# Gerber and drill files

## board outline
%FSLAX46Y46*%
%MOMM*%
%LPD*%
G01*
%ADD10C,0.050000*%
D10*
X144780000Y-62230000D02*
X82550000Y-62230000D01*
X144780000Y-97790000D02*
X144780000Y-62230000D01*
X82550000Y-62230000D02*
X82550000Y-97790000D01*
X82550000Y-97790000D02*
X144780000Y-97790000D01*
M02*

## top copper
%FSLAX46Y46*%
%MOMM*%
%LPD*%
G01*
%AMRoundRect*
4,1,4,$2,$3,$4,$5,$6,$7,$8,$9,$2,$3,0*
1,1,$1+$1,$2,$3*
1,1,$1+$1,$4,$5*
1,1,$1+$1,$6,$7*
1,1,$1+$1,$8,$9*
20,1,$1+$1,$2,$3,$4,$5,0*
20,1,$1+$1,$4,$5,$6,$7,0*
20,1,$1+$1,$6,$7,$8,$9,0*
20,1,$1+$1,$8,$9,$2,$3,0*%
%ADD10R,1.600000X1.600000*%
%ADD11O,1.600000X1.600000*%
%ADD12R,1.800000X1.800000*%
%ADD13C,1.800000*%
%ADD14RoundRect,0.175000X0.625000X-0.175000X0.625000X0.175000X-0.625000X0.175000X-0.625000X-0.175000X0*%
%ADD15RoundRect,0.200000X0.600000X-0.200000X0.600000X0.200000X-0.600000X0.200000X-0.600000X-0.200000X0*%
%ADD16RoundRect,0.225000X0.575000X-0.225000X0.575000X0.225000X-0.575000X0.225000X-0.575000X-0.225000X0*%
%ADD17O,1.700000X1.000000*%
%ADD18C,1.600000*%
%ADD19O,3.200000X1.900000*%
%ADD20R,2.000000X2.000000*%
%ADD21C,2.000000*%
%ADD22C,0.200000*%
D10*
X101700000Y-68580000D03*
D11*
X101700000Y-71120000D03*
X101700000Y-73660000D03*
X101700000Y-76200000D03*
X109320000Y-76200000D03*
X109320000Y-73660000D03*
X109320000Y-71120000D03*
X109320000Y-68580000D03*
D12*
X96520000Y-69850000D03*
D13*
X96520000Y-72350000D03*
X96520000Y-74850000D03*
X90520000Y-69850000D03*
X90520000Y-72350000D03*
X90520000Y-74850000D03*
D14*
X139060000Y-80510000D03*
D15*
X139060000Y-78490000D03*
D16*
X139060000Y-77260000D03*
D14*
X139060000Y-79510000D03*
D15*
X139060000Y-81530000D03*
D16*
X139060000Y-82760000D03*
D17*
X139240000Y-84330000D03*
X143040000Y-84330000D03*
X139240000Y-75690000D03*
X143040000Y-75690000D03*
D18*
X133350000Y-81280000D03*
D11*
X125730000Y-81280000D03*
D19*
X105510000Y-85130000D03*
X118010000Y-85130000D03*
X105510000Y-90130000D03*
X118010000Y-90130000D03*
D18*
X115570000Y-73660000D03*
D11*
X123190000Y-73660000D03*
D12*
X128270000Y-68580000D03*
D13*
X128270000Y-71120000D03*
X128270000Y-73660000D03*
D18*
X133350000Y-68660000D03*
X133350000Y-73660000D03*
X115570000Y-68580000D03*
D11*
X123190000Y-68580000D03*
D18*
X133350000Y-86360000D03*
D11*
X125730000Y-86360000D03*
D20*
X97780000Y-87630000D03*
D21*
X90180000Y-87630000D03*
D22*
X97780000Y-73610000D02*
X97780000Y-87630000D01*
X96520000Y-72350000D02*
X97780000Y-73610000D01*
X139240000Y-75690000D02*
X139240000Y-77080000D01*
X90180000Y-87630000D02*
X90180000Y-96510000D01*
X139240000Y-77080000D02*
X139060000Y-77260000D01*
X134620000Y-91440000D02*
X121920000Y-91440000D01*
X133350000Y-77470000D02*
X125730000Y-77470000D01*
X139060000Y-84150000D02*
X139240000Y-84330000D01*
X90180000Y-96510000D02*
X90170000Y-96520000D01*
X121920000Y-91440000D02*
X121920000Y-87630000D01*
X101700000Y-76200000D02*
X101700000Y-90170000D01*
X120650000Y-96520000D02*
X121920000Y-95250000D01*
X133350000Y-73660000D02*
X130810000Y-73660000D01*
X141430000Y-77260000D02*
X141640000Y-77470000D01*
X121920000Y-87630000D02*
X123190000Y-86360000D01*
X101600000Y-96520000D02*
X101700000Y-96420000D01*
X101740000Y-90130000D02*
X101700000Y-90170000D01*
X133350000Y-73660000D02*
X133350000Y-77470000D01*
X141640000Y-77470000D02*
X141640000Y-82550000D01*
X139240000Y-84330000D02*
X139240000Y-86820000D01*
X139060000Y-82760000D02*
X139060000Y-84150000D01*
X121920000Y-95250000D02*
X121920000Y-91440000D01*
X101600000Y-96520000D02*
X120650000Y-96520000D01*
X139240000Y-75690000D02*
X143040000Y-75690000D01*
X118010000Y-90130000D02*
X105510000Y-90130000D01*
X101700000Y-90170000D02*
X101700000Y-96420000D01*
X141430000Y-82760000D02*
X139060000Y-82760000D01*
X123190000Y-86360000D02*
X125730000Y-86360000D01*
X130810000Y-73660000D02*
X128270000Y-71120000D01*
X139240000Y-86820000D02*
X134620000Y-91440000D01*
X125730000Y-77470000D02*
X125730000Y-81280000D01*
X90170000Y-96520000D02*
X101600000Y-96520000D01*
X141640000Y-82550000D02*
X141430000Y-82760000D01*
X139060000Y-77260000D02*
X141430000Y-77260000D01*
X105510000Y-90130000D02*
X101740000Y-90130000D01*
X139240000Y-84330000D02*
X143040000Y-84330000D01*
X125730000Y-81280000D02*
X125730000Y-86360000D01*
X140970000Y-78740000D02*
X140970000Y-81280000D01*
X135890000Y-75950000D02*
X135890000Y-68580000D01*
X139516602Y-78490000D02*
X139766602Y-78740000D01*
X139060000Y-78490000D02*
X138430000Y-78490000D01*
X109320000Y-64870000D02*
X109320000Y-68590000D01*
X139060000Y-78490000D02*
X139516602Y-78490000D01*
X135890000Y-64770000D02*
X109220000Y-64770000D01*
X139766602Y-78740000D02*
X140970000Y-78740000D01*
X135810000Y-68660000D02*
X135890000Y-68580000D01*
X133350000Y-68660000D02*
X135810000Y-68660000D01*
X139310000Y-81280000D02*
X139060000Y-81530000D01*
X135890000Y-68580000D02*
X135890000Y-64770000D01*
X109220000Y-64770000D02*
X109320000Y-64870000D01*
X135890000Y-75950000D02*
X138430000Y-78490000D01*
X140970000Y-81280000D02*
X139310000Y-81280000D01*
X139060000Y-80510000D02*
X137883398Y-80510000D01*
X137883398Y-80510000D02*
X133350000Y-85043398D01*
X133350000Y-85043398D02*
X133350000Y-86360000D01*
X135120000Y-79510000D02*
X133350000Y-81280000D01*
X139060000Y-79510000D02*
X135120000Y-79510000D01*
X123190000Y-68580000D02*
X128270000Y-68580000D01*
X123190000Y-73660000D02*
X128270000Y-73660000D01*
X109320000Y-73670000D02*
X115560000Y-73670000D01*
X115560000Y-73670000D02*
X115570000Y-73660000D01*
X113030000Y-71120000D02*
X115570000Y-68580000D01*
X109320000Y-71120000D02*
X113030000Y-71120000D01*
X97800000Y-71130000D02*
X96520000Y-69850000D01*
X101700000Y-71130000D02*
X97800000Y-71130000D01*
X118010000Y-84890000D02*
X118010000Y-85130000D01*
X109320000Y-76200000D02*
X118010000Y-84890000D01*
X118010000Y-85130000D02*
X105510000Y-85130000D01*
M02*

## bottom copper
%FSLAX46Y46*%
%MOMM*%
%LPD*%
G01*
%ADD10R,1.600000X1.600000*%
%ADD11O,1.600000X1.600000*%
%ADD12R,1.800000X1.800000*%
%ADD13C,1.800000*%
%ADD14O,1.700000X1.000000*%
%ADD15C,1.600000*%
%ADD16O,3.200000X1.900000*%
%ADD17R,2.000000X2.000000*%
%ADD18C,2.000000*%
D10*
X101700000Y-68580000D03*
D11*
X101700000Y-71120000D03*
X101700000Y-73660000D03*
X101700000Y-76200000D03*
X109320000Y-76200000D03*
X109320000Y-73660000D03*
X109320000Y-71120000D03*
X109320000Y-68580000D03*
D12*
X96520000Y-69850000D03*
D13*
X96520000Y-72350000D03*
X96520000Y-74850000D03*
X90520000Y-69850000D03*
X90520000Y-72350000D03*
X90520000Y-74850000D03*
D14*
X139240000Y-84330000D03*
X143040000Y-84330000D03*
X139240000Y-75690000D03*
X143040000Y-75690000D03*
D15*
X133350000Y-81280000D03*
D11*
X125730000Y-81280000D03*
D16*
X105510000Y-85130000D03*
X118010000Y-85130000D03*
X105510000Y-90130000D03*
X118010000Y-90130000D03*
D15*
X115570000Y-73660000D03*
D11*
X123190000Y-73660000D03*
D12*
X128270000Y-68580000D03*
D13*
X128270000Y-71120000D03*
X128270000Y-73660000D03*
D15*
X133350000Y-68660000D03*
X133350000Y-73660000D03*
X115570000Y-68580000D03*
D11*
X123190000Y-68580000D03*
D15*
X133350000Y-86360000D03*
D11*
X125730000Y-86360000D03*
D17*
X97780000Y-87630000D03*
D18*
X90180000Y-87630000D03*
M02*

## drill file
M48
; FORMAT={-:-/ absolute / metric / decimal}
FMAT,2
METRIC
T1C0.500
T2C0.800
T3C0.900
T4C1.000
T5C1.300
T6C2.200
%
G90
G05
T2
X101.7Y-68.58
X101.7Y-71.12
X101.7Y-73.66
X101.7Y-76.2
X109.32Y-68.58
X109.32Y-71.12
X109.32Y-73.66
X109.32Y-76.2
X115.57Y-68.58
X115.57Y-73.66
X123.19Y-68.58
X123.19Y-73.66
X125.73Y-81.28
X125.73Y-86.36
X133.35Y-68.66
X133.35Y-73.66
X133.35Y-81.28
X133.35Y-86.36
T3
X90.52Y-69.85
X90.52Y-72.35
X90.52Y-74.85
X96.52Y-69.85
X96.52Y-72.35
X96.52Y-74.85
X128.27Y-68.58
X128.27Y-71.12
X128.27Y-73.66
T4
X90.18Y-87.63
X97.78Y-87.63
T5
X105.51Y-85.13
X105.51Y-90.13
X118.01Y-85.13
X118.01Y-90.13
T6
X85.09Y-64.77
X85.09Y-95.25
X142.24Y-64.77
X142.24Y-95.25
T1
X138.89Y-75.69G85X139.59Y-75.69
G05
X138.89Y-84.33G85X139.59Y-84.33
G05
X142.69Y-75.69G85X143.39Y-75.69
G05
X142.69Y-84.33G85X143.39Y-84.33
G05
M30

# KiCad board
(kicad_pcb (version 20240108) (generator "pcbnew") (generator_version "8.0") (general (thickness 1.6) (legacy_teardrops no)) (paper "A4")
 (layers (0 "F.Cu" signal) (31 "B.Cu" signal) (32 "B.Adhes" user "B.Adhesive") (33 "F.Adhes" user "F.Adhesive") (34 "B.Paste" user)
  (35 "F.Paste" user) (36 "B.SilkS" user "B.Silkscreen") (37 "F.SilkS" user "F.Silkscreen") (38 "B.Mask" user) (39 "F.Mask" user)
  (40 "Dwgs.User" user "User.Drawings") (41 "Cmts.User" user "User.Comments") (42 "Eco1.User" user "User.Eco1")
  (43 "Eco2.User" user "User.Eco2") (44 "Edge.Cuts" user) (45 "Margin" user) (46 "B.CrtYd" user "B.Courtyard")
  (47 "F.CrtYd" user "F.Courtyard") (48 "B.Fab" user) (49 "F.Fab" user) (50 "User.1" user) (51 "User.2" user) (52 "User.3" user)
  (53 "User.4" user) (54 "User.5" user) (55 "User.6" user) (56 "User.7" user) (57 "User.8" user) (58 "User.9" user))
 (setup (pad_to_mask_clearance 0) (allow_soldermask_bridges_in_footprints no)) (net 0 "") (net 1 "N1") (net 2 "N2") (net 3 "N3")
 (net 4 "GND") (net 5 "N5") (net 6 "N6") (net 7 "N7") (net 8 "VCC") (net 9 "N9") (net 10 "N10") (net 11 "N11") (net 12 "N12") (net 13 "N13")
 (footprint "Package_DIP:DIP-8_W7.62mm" (layer "F.Cu") (at 101.7 68.58)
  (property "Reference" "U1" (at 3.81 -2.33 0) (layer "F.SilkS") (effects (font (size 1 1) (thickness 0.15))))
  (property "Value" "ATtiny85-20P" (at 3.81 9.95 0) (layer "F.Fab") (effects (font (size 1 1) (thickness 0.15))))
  (pad "1" thru_hole rect (at 0 0) (size 1.6 1.6) (drill 0.8) (layers "*.Cu" "*.Mask") (remove_unused_layers no) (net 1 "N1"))
  (pad "2" thru_hole oval (at 0 2.54) (size 1.6 1.6) (drill 0.8) (layers "*.Cu" "*.Mask") (remove_unused_layers no) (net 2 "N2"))
  (pad "3" thru_hole oval (at 0 5.08) (size 1.6 1.6) (drill 0.8) (layers "*.Cu" "*.Mask") (remove_unused_layers no) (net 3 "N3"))
  (pad "4" thru_hole oval (at 0 7.62) (size 1.6 1.6) (drill 0.8) (layers "*.Cu" "*.Mask") (remove_unused_layers no) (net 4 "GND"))
  (pad "5" thru_hole oval (at 7.62 7.62) (size 1.6 1.6) (drill 0.8) (layers "*.Cu" "*.Mask") (remove_unused_layers no) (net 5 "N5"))
  (pad "6" thru_hole oval (at 7.62 5.08) (size 1.6 1.6) (drill 0.8) (layers "*.Cu" "*.Mask") (remove_unused_layers no) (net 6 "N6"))
  (pad "7" thru_hole oval (at 7.62 2.54) (size 1.6 1.6) (drill 0.8) (layers "*.Cu" "*.Mask") (remove_unused_layers no) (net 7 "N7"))
  (pad "8" thru_hole oval (at 7.62 0) (size 1.6 1.6) (drill 0.8) (layers "*.Cu" "*.Mask") (remove_unused_layers no) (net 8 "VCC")))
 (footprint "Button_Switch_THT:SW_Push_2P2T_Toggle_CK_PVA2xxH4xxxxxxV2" (layer "F.Cu") (at 96.52 69.85 -90)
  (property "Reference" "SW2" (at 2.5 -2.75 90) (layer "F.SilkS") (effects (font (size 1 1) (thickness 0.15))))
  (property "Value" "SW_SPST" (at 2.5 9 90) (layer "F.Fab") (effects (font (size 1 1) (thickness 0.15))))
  (pad "1" thru_hole rect (at 0 0 270) (size 1.8 1.8) (drill 0.9) (layers "*.Cu" "*.Mask") (remove_unused_layers no) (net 2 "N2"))
  (pad "2" thru_hole circle (at 2.5 0 270) (size 1.8 1.8) (drill 0.9) (layers "*.Cu" "*.Mask") (remove_unused_layers no) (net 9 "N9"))
  (pad "3" thru_hole circle (at 5 0 270) (size 1.8 1.8) (drill 0.9) (layers "*.Cu" "*.Mask") (remove_unused_layers no))
  (pad "4" thru_hole circle (at 0 6 270) (size 1.8 1.8) (drill 0.9) (layers "*.Cu" "*.Mask") (remove_unused_layers no))
  (pad "5" thru_hole circle (at 2.5 6 270) (size 1.8 1.8) (drill 0.9) (layers "*.Cu" "*.Mask") (remove_unused_layers no))
  (pad "6" thru_hole circle (at 5 6 270) (size 1.8 1.8) (drill 0.9) (layers "*.Cu" "*.Mask") (remove_unused_layers no)))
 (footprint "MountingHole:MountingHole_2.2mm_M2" (layer "F.Cu") (at 142.24 95.25)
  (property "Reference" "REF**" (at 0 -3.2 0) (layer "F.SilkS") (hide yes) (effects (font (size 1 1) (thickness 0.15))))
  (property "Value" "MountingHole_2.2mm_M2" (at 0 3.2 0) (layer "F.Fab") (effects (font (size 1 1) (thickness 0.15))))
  (pad "" np_thru_hole circle (at 0 0) (size 2.2 2.2) (drill 2.2) (layers "*.Cu" "*.Mask")))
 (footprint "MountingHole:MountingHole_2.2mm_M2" (layer "F.Cu") (at 142.24 64.77)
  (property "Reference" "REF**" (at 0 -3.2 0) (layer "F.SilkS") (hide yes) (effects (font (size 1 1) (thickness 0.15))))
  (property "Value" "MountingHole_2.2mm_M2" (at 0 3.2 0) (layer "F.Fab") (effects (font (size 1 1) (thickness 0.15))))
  (pad "" np_thru_hole circle (at 0 0) (size 2.2 2.2) (drill 2.2) (layers "*.Cu" "*.Mask")))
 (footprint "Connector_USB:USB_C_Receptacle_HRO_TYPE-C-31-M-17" (layer "F.Cu") (at 142.24 80.01 90)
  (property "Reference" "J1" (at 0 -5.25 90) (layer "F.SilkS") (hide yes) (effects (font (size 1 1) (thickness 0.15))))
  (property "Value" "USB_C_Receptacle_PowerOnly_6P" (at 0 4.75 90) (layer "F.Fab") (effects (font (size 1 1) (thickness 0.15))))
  (pad "A5" smd roundrect (at -0.5 -3.18 90) (size 0.7 1.6) (layers "F.Cu" "F.Paste" "F.Mask") (roundrect_rratio 0.25) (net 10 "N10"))
  (pad "A9" smd roundrect (at 1.52 -3.18 90) (size 0.8 1.6) (layers "F.Cu" "F.Paste" "F.Mask") (roundrect_rratio 0.25) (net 8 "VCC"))
  (pad "A12" smd roundrect (at 2.75 -3.18 90) (size 0.9 1.6) (layers "F.Cu" "F.Paste" "F.Mask") (roundrect_rratio 0.25) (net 4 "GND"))
  (pad "B5" smd roundrect (at 0.5 -3.18 90) (size 0.7 1.6) (layers "F.Cu" "F.Paste" "F.Mask") (roundrect_rratio 0.25) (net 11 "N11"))
  (pad "B9" smd roundrect (at -1.52 -3.18 90) (size 0.8 1.6) (layers "F.Cu" "F.Paste" "F.Mask") (roundrect_rratio 0.25) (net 8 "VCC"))
  (pad "B12" smd roundrect (at -2.75 -3.18 90) (size 0.9 1.6) (layers "F.Cu" "F.Paste" "F.Mask") (roundrect_rratio 0.25) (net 4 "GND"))
  (pad "S1" thru_hole oval (at -4.32 -3 90) (size 1 1.7) (drill oval 0.5 1.2) (layers "*.Cu" "*.Mask") (remove_unused_layers no)
   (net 4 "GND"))
  (pad "S1" thru_hole oval (at -4.32 0.8 90) (size 1 1.7) (drill oval 0.5 1.2) (layers "*.Cu" "*.Mask") (remove_unused_layers no)
   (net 4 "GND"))
  (pad "S1" thru_hole oval (at 4.32 -3 90) (size 1 1.7) (drill oval 0.5 1.2) (layers "*.Cu" "*.Mask") (remove_unused_layers no)
   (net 4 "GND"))
  (pad "S1" thru_hole oval (at 4.32 0.8 90) (size 1 1.7) (drill oval 0.5 1.2) (layers "*.Cu" "*.Mask") (remove_unused_layers no)
   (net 4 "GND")))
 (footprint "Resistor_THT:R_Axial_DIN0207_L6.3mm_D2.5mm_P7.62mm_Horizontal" (layer "F.Cu") (at 133.35 81.28 180)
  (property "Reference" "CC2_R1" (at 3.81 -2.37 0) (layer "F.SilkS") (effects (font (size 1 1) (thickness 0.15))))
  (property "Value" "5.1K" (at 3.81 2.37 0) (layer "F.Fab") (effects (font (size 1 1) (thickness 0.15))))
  (pad "1" thru_hole circle (at 0 0 180) (size 1.6 1.6) (drill 0.8) (layers "*.Cu" "*.Mask") (remove_unused_layers no) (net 11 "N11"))
  (pad "2" thru_hole oval (at 7.62 0 180) (size 1.6 1.6) (drill 0.8) (layers "*.Cu" "*.Mask") (remove_unused_layers no) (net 4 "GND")))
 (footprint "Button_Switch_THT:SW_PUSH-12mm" (layer "F.Cu") (at 105.51 85.13)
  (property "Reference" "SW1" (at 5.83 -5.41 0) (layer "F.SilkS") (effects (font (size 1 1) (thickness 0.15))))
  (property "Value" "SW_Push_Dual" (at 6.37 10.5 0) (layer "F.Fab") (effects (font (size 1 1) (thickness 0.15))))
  (pad "1" thru_hole oval (at 0 0) (size 3.2 1.9) (drill 1.3) (layers "*.Cu" "*.Mask") (remove_unused_layers no) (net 5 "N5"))
  (pad "1" thru_hole oval (at 12.5 0) (size 3.2 1.9) (drill 1.3) (layers "*.Cu" "*.Mask") (remove_unused_layers no) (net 5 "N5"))
  (pad "2" thru_hole oval (at 0 5) (size 3.2 1.9) (drill 1.3) (layers "*.Cu" "*.Mask") (remove_unused_layers no) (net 4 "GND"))
  (pad "2" thru_hole oval (at 12.5 5) (size 3.2 1.9) (drill 1.3) (layers "*.Cu" "*.Mask") (remove_unused_layers no) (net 4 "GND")))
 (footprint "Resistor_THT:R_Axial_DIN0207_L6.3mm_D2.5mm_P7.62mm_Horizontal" (layer "F.Cu") (at 115.57 73.66)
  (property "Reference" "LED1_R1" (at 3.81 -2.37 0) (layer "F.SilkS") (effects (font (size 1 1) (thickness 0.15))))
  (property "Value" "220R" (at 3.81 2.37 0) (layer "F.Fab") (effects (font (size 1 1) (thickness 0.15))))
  (pad "1" thru_hole circle (at 0 0) (size 1.6 1.6) (drill 0.8) (layers "*.Cu" "*.Mask") (remove_unused_layers no) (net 6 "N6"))
  (pad "2" thru_hole oval (at 7.62 0) (size 1.6 1.6) (drill 0.8) (layers "*.Cu" "*.Mask") (remove_unused_layers no) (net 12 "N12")))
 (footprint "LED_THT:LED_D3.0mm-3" (layer "F.Cu") (at 128.27 68.58 -90)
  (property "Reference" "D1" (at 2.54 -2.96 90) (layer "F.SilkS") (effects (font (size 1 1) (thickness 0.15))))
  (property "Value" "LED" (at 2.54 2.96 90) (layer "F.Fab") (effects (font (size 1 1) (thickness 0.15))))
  (pad "1" thru_hole rect (at 0 0 270) (size 1.8 1.8) (drill 0.9) (layers "*.Cu" "*.Mask") (remove_unused_layers no) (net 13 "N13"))
  (pad "2" thru_hole circle (at 2.54 0 270) (size 1.8 1.8) (drill 0.9) (layers "*.Cu" "*.Mask") (remove_unused_layers no) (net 4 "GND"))
  (pad "3" thru_hole circle (at 5.08 0 270) (size 1.8 1.8) (drill 0.9) (layers "*.Cu" "*.Mask") (remove_unused_layers no) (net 12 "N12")))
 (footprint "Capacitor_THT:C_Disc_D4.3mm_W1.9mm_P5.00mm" (layer "F.Cu") (at 133.35 68.66 -90)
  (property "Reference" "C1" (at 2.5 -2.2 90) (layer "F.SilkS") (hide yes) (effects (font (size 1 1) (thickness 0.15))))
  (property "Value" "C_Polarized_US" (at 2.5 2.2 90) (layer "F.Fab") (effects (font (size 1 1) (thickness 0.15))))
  (pad "1" thru_hole circle (at 0 0 270) (size 1.6 1.6) (drill 0.8) (layers "*.Cu" "*.Mask") (remove_unused_layers no) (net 8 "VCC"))
  (pad "2" thru_hole circle (at 5 0 270) (size 1.6 1.6) (drill 0.8) (layers "*.Cu" "*.Mask") (remove_unused_layers no) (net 4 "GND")))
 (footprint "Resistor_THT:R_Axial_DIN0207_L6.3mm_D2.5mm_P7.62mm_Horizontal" (layer "F.Cu") (at 115.57 68.58)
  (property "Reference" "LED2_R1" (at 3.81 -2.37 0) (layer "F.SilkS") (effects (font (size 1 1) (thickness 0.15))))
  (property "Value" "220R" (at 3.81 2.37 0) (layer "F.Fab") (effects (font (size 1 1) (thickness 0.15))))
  (pad "1" thru_hole circle (at 0 0) (size 1.6 1.6) (drill 0.8) (layers "*.Cu" "*.Mask") (remove_unused_layers no) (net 7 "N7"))
  (pad "2" thru_hole oval (at 7.62 0) (size 1.6 1.6) (drill 0.8) (layers "*.Cu" "*.Mask") (remove_unused_layers no) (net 13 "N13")))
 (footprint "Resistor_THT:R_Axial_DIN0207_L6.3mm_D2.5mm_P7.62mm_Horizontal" (layer "F.Cu") (at 133.35 86.36 180)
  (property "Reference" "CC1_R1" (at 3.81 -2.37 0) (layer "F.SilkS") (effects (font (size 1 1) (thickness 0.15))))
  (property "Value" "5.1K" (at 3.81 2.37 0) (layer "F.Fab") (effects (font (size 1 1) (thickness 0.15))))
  (pad "1" thru_hole circle (at 0 0 180) (size 1.6 1.6) (drill 0.8) (layers "*.Cu" "*.Mask") (remove_unused_layers no) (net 10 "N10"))
  (pad "2" thru_hole oval (at 7.62 0 180) (size 1.6 1.6) (drill 0.8) (layers "*.Cu" "*.Mask") (remove_unused_layers no) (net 4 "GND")))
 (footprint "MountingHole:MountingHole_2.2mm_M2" (layer "F.Cu") (at 85.09 64.77)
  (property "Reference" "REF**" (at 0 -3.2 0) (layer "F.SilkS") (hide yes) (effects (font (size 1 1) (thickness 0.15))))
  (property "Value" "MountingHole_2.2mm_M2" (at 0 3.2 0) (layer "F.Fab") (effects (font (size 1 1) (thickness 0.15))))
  (pad "" np_thru_hole circle (at 0 0) (size 2.2 2.2) (drill 2.2) (layers "*.Cu" "*.Mask")))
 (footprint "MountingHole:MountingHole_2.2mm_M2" (layer "F.Cu") (at 85.09 95.25)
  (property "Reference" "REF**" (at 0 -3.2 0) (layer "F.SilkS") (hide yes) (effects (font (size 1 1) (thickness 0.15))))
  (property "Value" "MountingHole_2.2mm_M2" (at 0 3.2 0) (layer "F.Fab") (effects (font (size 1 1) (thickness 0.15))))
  (pad "" np_thru_hole circle (at 0 0) (size 2.2 2.2) (drill 2.2) (layers "*.Cu" "*.Mask")))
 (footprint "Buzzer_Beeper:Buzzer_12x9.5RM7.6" (layer "F.Cu") (at 97.78 87.63 180)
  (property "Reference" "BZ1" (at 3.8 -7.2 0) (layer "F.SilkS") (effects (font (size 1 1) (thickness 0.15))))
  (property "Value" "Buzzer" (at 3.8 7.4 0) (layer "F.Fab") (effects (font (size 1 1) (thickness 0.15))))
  (pad "1" thru_hole rect (at 0 0 180) (size 2 2) (drill 1) (layers "*.Cu" "*.Mask") (remove_unused_layers no) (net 9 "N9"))
  (pad "2" thru_hole circle (at 7.6 0 180) (size 2 2) (drill 1) (layers "*.Cu" "*.Mask") (remove_unused_layers no) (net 4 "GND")))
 (gr_line (start 144.78 62.23) (end 82.55 62.23) (stroke (width 0.05) (type default)) (layer "Edge.Cuts"))
 (gr_line (start 144.78 97.79) (end 144.78 62.23) (stroke (width 0.05) (type default)) (layer "Edge.Cuts"))
 (gr_line (start 82.55 62.23) (end 82.55 97.79) (stroke (width 0.05) (type default)) (layer "Edge.Cuts"))
 (gr_line (start 82.55 97.79) (end 144.78 97.79) (stroke (width 0.05) (type default)) (layer "Edge.Cuts"))
 (segment (start 97.78 73.61) (end 97.78 87.63) (width 0.2) (layer "F.Cu") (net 9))
 (segment (start 96.52 72.35) (end 97.78 73.61) (width 0.2) (layer "F.Cu") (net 9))
 (segment (start 139.24 75.69) (end 139.24 77.08) (width 0.2) (layer "F.Cu") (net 4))
 (segment (start 90.18 87.63) (end 90.18 96.51) (width 0.2) (layer "F.Cu") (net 4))
 (segment (start 139.24 77.08) (end 139.06 77.26) (width 0.2) (layer "F.Cu") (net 4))
 (segment (start 134.62 91.44) (end 121.92 91.44) (width 0.2) (layer "F.Cu") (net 4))
 (segment (start 133.35 77.47) (end 125.73 77.47) (width 0.2) (layer "F.Cu") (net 4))
 (segment (start 139.06 84.15) (end 139.24 84.33) (width 0.2) (layer "F.Cu") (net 4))
 (segment (start 90.18 96.51) (end 90.17 96.52) (width 0.2) (layer "F.Cu") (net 4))
 (segment (start 121.92 91.44) (end 121.92 87.63) (width 0.2) (layer "F.Cu") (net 4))
 (segment (start 101.7 76.2) (end 101.7 90.17) (width 0.2) (layer "F.Cu") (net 4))
 (segment (start 120.65 96.52) (end 121.92 95.25) (width 0.2) (layer "F.Cu") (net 4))
 (segment (start 133.35 73.66) (end 130.81 73.66) (width 0.2) (layer "F.Cu") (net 4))
 (segment (start 141.43 77.26) (end 141.64 77.47) (width 0.2) (layer "F.Cu") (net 4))
 (segment (start 121.92 87.63) (end 123.19 86.36) (width 0.2) (layer "F.Cu") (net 4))
 (segment (start 101.6 96.52) (end 101.7 96.42) (width 0.2) (layer "F.Cu") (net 4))
 (segment (start 101.74 90.13) (end 101.7 90.17) (width 0.2) (layer "F.Cu") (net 4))
 (segment (start 133.35 73.66) (end 133.35 77.47) (width 0.2) (layer "F.Cu") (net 4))
 (segment (start 141.64 77.47) (end 141.64 82.55) (width 0.2) (layer "F.Cu") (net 4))
 (segment (start 139.24 84.33) (end 139.24 86.82) (width 0.2) (layer "F.Cu") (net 4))
 (segment (start 139.06 82.76) (end 139.06 84.15) (width 0.2) (layer "F.Cu") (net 4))
 (segment (start 121.92 95.25) (end 121.92 91.44) (width 0.2) (layer "F.Cu") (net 4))
 (segment (start 101.6 96.52) (end 120.65 96.52) (width 0.2) (layer "F.Cu") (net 4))
 (segment (start 139.24 75.69) (end 143.04 75.69) (width 0.2) (layer "F.Cu") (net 4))
 (segment (start 118.01 90.13) (end 105.51 90.13) (width 0.2) (layer "F.Cu") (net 4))
 (segment (start 101.7 90.17) (end 101.7 96.42) (width 0.2) (layer "F.Cu") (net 4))
 (segment (start 141.43 82.76) (end 139.06 82.76) (width 0.2) (layer "F.Cu") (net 4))
 (segment (start 123.19 86.36) (end 125.73 86.36) (width 0.2) (layer "F.Cu") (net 4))
 (segment (start 130.81 73.66) (end 128.27 71.12) (width 0.2) (layer "F.Cu") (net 4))
 (segment (start 139.24 86.82) (end 134.62 91.44) (width 0.2) (layer "F.Cu") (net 4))
 (segment (start 125.73 77.47) (end 125.73 81.28) (width 0.2) (layer "F.Cu") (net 4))
 (segment (start 90.17 96.52) (end 101.6 96.52) (width 0.2) (layer "F.Cu") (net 4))
 (segment (start 141.64 82.55) (end 141.43 82.76) (width 0.2) (layer "F.Cu") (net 4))
 (segment (start 139.06 77.26) (end 141.43 77.26) (width 0.2) (layer "F.Cu") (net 4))
 (segment (start 105.51 90.13) (end 101.74 90.13) (width 0.2) (layer "F.Cu") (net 4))
 (segment (start 139.24 84.33) (end 143.04 84.33) (width 0.2) (layer "F.Cu") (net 4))
 (segment (start 125.73 81.28) (end 125.73 86.36) (width 0.2) (layer "F.Cu") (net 4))
 (segment (start 140.97 78.74) (end 140.97 81.28) (width 0.2) (layer "F.Cu") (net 8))
 (segment (start 135.89 75.95) (end 135.89 68.58) (width 0.2) (layer "F.Cu") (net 8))
 (segment (start 139.516602 78.49) (end 139.766602 78.74) (width 0.2) (layer "F.Cu") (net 8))
 (segment (start 139.06 78.49) (end 138.43 78.49) (width 0.2) (layer "F.Cu") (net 8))
 (segment (start 109.32 64.87) (end 109.32 68.59) (width 0.2) (layer "F.Cu") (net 8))
 (segment (start 139.06 78.49) (end 139.516602 78.49) (width 0.2) (layer "F.Cu") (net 8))
 (segment (start 135.89 64.77) (end 109.22 64.77) (width 0.2) (layer "F.Cu") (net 8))
 (segment (start 139.766602 78.74) (end 140.97 78.74) (width 0.2) (layer "F.Cu") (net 8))
 (segment (start 135.81 68.66) (end 135.89 68.58) (width 0.2) (layer "F.Cu") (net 8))
 (segment (start 133.35 68.66) (end 135.81 68.66) (width 0.2) (layer "F.Cu") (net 8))
 (segment (start 139.31 81.28) (end 139.06 81.53) (width 0.2) (layer "F.Cu") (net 8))
 (segment (start 135.89 68.58) (end 135.89 64.77) (width 0.2) (layer "F.Cu") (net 8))
 (segment (start 109.22 64.77) (end 109.32 64.87) (width 0.2) (layer "F.Cu") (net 8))
 (segment (start 135.89 75.95) (end 138.43 78.49) (width 0.2) (layer "F.Cu") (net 8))
 (segment (start 140.97 81.28) (end 139.31 81.28) (width 0.2) (layer "F.Cu") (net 8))
 (segment (start 139.06 80.51) (end 137.883398 80.51) (width 0.2) (layer "F.Cu") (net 10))
 (segment (start 137.883398 80.51) (end 133.35 85.043398) (width 0.2) (layer "F.Cu") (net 10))
 (segment (start 133.35 85.043398) (end 133.35 86.36) (width 0.2) (layer "F.Cu") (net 10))
 (segment (start 135.12 79.51) (end 133.35 81.28) (width 0.2) (layer "F.Cu") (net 11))
 (segment (start 139.06 79.51) (end 135.12 79.51) (width 0.2) (layer "F.Cu") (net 11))
 (segment (start 123.19 68.58) (end 128.27 68.58) (width 0.2) (layer "F.Cu") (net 13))
 (segment (start 123.19 73.66) (end 128.27 73.66) (width 0.2) (layer "F.Cu") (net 12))
 (segment (start 109.32 73.67) (end 115.56 73.67) (width 0.2) (layer "F.Cu") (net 6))
 (segment (start 115.56 73.67) (end 115.57 73.66) (width 0.2) (layer "F.Cu") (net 6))
 (segment (start 113.03 71.12) (end 115.57 68.58) (width 0.2) (layer "F.Cu") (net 7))
 (segment (start 109.32 71.12) (end 113.03 71.12) (width 0.2) (layer "F.Cu") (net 7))
 (segment (start 97.8 71.13) (end 96.52 69.85) (width 0.2) (layer "F.Cu") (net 2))
 (segment (start 101.7 71.13) (end 97.8 71.13) (width 0.2) (layer "F.Cu") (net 2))
 (segment (start 118.01 84.89) (end 118.01 85.13) (width 0.2) (layer "F.Cu") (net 5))
 (segment (start 109.32 76.2) (end 118.01 84.89) (width 0.2) (layer "F.Cu") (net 5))
 (segment (start 118.01 85.13) (end 105.51 85.13) (width 0.2) (layer "F.Cu") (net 5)))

